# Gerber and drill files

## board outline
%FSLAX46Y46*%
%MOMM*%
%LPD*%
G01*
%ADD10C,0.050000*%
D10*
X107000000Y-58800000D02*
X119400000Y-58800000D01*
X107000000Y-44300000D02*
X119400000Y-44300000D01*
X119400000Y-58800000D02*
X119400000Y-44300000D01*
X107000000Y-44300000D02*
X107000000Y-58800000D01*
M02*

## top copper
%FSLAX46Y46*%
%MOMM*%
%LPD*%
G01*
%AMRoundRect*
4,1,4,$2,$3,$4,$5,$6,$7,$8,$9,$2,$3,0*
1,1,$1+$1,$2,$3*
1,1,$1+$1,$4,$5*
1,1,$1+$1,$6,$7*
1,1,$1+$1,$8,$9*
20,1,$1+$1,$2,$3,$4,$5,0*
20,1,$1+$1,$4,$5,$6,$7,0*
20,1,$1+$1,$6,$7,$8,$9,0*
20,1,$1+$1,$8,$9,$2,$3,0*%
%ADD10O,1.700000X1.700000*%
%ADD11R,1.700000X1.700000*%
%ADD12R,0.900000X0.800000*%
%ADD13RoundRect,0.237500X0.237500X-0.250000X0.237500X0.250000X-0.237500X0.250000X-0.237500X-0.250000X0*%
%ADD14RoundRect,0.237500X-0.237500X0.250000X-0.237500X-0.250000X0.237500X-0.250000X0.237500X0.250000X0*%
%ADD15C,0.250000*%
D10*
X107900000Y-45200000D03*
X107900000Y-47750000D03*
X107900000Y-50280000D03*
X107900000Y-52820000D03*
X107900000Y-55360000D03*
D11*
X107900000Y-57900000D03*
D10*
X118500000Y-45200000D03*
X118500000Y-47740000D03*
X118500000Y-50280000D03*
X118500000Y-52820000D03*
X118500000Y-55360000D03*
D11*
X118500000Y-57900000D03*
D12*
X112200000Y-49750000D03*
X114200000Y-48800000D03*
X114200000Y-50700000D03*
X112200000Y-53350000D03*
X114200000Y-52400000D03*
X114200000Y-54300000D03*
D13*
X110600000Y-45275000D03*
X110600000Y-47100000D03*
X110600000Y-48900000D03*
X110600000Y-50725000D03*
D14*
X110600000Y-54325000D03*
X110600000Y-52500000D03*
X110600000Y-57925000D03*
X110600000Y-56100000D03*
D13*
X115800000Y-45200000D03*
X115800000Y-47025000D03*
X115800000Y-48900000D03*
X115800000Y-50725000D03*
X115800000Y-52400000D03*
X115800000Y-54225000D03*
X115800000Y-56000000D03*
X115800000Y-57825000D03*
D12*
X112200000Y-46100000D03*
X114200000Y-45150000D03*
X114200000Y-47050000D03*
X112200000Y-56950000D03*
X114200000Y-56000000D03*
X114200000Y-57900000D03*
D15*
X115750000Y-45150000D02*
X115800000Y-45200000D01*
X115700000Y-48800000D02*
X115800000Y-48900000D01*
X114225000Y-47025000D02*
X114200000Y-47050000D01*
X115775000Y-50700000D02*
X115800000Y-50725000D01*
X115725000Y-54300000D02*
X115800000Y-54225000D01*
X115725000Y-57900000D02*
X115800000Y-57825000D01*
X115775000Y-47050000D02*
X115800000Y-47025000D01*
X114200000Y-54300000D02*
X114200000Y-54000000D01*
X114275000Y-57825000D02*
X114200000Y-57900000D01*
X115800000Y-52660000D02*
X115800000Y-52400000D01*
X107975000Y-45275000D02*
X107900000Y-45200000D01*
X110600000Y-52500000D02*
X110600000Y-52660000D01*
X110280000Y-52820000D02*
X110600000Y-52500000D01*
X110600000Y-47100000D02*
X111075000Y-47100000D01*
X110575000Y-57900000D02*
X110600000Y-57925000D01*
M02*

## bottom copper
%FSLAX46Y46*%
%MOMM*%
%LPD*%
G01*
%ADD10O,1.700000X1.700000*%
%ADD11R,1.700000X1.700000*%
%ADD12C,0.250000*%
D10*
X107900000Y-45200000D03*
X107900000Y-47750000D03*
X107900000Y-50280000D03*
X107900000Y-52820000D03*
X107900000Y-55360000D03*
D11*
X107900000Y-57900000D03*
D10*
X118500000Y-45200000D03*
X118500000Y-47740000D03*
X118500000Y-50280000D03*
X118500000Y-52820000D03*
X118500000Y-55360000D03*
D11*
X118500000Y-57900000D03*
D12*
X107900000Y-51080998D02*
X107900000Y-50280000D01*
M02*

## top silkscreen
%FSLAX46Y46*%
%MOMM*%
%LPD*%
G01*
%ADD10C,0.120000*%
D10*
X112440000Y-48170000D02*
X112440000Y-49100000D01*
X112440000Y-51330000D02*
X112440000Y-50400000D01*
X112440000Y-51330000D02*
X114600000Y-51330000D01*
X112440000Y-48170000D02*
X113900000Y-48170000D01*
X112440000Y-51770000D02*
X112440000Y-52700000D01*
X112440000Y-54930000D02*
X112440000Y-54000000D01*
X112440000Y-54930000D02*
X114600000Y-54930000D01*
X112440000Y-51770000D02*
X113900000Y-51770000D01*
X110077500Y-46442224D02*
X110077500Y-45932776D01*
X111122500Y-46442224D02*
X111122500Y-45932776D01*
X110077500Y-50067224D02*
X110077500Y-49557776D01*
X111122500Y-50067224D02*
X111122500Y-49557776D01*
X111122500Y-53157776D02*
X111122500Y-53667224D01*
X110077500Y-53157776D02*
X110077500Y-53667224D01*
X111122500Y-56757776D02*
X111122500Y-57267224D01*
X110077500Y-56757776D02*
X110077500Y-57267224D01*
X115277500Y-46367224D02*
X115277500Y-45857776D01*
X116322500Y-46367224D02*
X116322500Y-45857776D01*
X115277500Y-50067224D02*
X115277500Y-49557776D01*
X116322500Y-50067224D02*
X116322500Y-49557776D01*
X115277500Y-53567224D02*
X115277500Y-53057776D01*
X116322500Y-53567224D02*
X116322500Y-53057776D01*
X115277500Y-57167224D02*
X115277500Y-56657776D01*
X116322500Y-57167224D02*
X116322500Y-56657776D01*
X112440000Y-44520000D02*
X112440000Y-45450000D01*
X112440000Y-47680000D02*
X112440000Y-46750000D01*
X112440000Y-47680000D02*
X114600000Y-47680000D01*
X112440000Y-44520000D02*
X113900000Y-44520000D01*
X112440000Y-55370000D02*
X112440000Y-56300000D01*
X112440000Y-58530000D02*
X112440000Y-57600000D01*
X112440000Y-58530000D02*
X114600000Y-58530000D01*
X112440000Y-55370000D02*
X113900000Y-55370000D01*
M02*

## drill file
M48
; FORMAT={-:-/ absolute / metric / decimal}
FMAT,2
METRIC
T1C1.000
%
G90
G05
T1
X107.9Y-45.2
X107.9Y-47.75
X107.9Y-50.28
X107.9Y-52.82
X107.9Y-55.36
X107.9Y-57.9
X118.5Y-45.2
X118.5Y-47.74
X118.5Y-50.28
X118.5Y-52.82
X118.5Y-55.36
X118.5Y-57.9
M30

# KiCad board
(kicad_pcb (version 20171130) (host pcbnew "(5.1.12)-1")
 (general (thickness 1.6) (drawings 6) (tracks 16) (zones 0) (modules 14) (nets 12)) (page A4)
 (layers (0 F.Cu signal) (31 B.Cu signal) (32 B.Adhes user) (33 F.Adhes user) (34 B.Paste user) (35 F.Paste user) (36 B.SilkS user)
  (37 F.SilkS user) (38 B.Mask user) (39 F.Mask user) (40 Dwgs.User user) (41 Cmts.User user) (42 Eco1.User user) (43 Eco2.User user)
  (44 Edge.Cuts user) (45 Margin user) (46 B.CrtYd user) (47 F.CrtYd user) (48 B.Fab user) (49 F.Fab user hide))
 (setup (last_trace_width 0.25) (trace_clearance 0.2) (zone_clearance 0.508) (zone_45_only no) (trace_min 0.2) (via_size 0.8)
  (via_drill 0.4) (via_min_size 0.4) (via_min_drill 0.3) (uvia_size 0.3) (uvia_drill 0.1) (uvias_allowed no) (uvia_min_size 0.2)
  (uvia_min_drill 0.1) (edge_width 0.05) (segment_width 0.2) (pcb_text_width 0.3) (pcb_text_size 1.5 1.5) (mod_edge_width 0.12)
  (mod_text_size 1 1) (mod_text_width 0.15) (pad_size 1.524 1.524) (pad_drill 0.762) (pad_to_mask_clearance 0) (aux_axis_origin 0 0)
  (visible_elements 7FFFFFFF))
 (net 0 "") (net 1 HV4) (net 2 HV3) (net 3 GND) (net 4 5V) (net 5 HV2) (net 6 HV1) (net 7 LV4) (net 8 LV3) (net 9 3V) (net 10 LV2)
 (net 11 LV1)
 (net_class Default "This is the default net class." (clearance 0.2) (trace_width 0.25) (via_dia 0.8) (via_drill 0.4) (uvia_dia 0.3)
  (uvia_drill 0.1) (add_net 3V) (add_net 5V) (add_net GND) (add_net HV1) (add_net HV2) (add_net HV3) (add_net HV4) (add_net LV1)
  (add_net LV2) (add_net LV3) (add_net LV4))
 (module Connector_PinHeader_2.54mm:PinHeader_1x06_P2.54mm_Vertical (layer B.Cu) (at 107.9 57.9)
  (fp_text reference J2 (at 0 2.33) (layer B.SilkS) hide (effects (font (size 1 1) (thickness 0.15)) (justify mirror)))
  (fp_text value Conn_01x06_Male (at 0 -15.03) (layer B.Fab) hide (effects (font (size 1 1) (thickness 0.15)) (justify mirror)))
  (pad 6 thru_hole oval (at 0 -12.7) (size 1.7 1.7) (drill 1) (layers *.Cu *.Mask) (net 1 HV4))
  (pad 5 thru_hole oval (at 0 -10.15) (size 1.7 1.7) (drill 1) (layers *.Cu *.Mask) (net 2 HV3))
  (pad 4 thru_hole oval (at 0 -7.62) (size 1.7 1.7) (drill 1) (layers *.Cu *.Mask) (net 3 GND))
  (pad 3 thru_hole oval (at 0 -5.08) (size 1.7 1.7) (drill 1) (layers *.Cu *.Mask) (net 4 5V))
  (pad 2 thru_hole oval (at 0 -2.54) (size 1.7 1.7) (drill 1) (layers *.Cu *.Mask) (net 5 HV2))
  (pad 1 thru_hole rect (at 0 0) (size 1.7 1.7) (drill 1) (layers *.Cu *.Mask) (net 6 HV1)))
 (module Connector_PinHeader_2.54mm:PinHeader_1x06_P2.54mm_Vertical (layer B.Cu) (at 118.5 57.9)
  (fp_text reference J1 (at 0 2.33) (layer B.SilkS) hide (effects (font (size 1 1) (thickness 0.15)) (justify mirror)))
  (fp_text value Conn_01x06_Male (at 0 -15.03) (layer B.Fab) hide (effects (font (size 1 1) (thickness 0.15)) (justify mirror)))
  (pad 6 thru_hole oval (at 0 -12.7) (size 1.7 1.7) (drill 1) (layers *.Cu *.Mask) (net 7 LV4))
  (pad 5 thru_hole oval (at 0 -10.16) (size 1.7 1.7) (drill 1) (layers *.Cu *.Mask) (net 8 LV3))
  (pad 4 thru_hole oval (at 0 -7.62) (size 1.7 1.7) (drill 1) (layers *.Cu *.Mask) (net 3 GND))
  (pad 3 thru_hole oval (at 0 -5.08) (size 1.7 1.7) (drill 1) (layers *.Cu *.Mask) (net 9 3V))
  (pad 2 thru_hole oval (at 0 -2.54) (size 1.7 1.7) (drill 1) (layers *.Cu *.Mask) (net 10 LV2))
  (pad 1 thru_hole rect (at 0 0) (size 1.7 1.7) (drill 1) (layers *.Cu *.Mask) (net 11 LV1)))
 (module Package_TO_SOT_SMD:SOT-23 (layer F.Cu) (at 113.2 49.75 180)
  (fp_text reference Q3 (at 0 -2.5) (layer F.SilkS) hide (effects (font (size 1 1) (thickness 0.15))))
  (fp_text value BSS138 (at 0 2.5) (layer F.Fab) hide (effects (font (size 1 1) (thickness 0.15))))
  (fp_line (start 0.76 1.58) (end 0.76 0.65) (layer F.SilkS) (width 0.12))
  (fp_line (start 0.76 -1.58) (end 0.76 -0.65) (layer F.SilkS) (width 0.12))
  (fp_line (start 0.76 -1.58) (end -1.4 -1.58) (layer F.SilkS) (width 0.12))
  (fp_line (start 0.76 1.58) (end -0.7 1.58) (layer F.SilkS) (width 0.12))
  (pad 3 smd rect (at 1 0 180) (size 0.9 0.8) (layers F.Cu F.Paste F.Mask) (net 2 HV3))
  (pad 2 smd rect (at -1 0.95 180) (size 0.9 0.8) (layers F.Cu F.Paste F.Mask) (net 8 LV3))
  (pad 1 smd rect (at -1 -0.95 180) (size 0.9 0.8) (layers F.Cu F.Paste F.Mask) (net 9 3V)))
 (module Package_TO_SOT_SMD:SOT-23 (layer F.Cu) (at 113.2 53.35 180)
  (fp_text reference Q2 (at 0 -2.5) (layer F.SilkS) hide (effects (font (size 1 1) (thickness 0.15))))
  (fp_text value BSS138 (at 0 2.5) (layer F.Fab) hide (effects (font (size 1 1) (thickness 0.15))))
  (fp_line (start 0.76 1.58) (end 0.76 0.65) (layer F.SilkS) (width 0.12))
  (fp_line (start 0.76 -1.58) (end 0.76 -0.65) (layer F.SilkS) (width 0.12))
  (fp_line (start 0.76 -1.58) (end -1.4 -1.58) (layer F.SilkS) (width 0.12))
  (fp_line (start 0.76 1.58) (end -0.7 1.58) (layer F.SilkS) (width 0.12))
  (pad 3 smd rect (at 1 0 180) (size 0.9 0.8) (layers F.Cu F.Paste F.Mask) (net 5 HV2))
  (pad 2 smd rect (at -1 0.95 180) (size 0.9 0.8) (layers F.Cu F.Paste F.Mask) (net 10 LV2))
  (pad 1 smd rect (at -1 -0.95 180) (size 0.9 0.8) (layers F.Cu F.Paste F.Mask) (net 9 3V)))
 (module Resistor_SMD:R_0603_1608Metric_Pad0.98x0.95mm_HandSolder (layer F.Cu) (at 110.6 46.1875 90)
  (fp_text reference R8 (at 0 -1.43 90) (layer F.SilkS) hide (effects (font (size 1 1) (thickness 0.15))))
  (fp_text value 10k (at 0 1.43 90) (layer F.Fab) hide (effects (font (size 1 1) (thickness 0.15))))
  (fp_line (start -0.254724 -0.5225) (end 0.254724 -0.5225) (layer F.SilkS) (width 0.12))
  (fp_line (start -0.254724 0.5225) (end 0.254724 0.5225) (layer F.SilkS) (width 0.12))
  (pad 2 smd roundrect (at 0.9125 0 90) (size 0.975 0.95) (layers F.Cu F.Paste F.Mask) (roundrect_rratio 0.25) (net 1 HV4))
  (pad 1 smd roundrect (at -0.9125 0 90) (size 0.975 0.95) (layers F.Cu F.Paste F.Mask) (roundrect_rratio 0.25) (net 4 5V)))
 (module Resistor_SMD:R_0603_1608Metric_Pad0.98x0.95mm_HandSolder (layer F.Cu) (at 110.6 49.8125 90)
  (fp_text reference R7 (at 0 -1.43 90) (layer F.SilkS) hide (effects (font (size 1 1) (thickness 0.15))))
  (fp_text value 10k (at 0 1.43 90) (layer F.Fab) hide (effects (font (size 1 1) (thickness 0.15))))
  (fp_line (start -0.254724 -0.5225) (end 0.254724 -0.5225) (layer F.SilkS) (width 0.12))
  (fp_line (start -0.254724 0.5225) (end 0.254724 0.5225) (layer F.SilkS) (width 0.12))
  (pad 2 smd roundrect (at 0.9125 0 90) (size 0.975 0.95) (layers F.Cu F.Paste F.Mask) (roundrect_rratio 0.25) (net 2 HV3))
  (pad 1 smd roundrect (at -0.9125 0 90) (size 0.975 0.95) (layers F.Cu F.Paste F.Mask) (roundrect_rratio 0.25) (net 4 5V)))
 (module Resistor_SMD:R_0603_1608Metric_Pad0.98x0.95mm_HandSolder (layer F.Cu) (at 110.6 53.4125 270)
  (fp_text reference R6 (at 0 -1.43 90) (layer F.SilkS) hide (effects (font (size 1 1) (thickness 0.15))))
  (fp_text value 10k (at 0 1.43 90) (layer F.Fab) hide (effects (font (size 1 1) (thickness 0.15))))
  (fp_line (start -0.254724 -0.5225) (end 0.254724 -0.5225) (layer F.SilkS) (width 0.12))
  (fp_line (start -0.254724 0.5225) (end 0.254724 0.5225) (layer F.SilkS) (width 0.12))
  (pad 2 smd roundrect (at 0.9125 0 270) (size 0.975 0.95) (layers F.Cu F.Paste F.Mask) (roundrect_rratio 0.25) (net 5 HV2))
  (pad 1 smd roundrect (at -0.9125 0 270) (size 0.975 0.95) (layers F.Cu F.Paste F.Mask) (roundrect_rratio 0.25) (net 4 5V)))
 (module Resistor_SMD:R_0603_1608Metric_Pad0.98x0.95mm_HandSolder (layer F.Cu) (at 110.6 57.0125 270)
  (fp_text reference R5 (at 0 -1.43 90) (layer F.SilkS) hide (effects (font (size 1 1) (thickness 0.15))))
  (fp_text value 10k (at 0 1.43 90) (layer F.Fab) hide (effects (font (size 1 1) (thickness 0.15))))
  (fp_line (start -0.254724 -0.5225) (end 0.254724 -0.5225) (layer F.SilkS) (width 0.12))
  (fp_line (start -0.254724 0.5225) (end 0.254724 0.5225) (layer F.SilkS) (width 0.12))
  (pad 2 smd roundrect (at 0.9125 0 270) (size 0.975 0.95) (layers F.Cu F.Paste F.Mask) (roundrect_rratio 0.25) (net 6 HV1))
  (pad 1 smd roundrect (at -0.9125 0 270) (size 0.975 0.95) (layers F.Cu F.Paste F.Mask) (roundrect_rratio 0.25) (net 4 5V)))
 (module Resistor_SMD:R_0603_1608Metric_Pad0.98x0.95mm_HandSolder (layer F.Cu) (at 115.8 46.1125 90)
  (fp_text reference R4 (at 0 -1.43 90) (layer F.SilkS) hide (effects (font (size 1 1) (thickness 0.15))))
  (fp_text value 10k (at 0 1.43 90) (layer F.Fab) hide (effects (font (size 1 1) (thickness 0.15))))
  (fp_line (start -0.254724 -0.5225) (end 0.254724 -0.5225) (layer F.SilkS) (width 0.12))
  (fp_line (start -0.254724 0.5225) (end 0.254724 0.5225) (layer F.SilkS) (width 0.12))
  (pad 2 smd roundrect (at 0.9125 0 90) (size 0.975 0.95) (layers F.Cu F.Paste F.Mask) (roundrect_rratio 0.25) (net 7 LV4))
  (pad 1 smd roundrect (at -0.9125 0 90) (size 0.975 0.95) (layers F.Cu F.Paste F.Mask) (roundrect_rratio 0.25) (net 9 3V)))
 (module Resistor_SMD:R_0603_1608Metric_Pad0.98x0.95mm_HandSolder (layer F.Cu) (at 115.8 49.8125 90)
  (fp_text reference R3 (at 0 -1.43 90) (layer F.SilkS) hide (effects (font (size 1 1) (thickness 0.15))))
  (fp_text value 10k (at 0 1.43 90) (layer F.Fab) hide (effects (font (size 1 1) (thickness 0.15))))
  (fp_line (start -0.254724 -0.5225) (end 0.254724 -0.5225) (layer F.SilkS) (width 0.12))
  (fp_line (start -0.254724 0.5225) (end 0.254724 0.5225) (layer F.SilkS) (width 0.12))
  (pad 2 smd roundrect (at 0.9125 0 90) (size 0.975 0.95) (layers F.Cu F.Paste F.Mask) (roundrect_rratio 0.25) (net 8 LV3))
  (pad 1 smd roundrect (at -0.9125 0 90) (size 0.975 0.95) (layers F.Cu F.Paste F.Mask) (roundrect_rratio 0.25) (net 9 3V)))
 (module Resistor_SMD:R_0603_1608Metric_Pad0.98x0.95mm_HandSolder (layer F.Cu) (at 115.8 53.3125 90)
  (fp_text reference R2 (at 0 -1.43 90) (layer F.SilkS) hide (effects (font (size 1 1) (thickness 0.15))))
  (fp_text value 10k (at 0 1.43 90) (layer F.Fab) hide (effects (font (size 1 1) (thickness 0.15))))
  (fp_line (start -0.254724 -0.5225) (end 0.254724 -0.5225) (layer F.SilkS) (width 0.12))
  (fp_line (start -0.254724 0.5225) (end 0.254724 0.5225) (layer F.SilkS) (width 0.12))
  (pad 2 smd roundrect (at 0.9125 0 90) (size 0.975 0.95) (layers F.Cu F.Paste F.Mask) (roundrect_rratio 0.25) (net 10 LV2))
  (pad 1 smd roundrect (at -0.9125 0 90) (size 0.975 0.95) (layers F.Cu F.Paste F.Mask) (roundrect_rratio 0.25) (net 9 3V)))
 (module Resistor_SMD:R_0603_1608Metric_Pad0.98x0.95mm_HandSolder (layer F.Cu) (at 115.8 56.9125 90)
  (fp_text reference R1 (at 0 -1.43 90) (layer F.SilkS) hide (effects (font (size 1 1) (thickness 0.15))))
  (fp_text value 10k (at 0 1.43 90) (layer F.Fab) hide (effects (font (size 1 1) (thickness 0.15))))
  (fp_line (start -0.254724 -0.5225) (end 0.254724 -0.5225) (layer F.SilkS) (width 0.12))
  (fp_line (start -0.254724 0.5225) (end 0.254724 0.5225) (layer F.SilkS) (width 0.12))
  (pad 2 smd roundrect (at 0.9125 0 90) (size 0.975 0.95) (layers F.Cu F.Paste F.Mask) (roundrect_rratio 0.25) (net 11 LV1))
  (pad 1 smd roundrect (at -0.9125 0 90) (size 0.975 0.95) (layers F.Cu F.Paste F.Mask) (roundrect_rratio 0.25) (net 9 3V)))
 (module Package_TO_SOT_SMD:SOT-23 (layer F.Cu) (at 113.2 46.1 180)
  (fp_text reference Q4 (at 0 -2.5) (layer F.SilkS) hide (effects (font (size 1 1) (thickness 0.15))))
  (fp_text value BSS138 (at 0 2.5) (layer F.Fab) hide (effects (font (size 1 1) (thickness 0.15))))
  (fp_line (start 0.76 1.58) (end 0.76 0.65) (layer F.SilkS) (width 0.12))
  (fp_line (start 0.76 -1.58) (end 0.76 -0.65) (layer F.SilkS) (width 0.12))
  (fp_line (start 0.76 -1.58) (end -1.4 -1.58) (layer F.SilkS) (width 0.12))
  (fp_line (start 0.76 1.58) (end -0.7 1.58) (layer F.SilkS) (width 0.12))
  (pad 3 smd rect (at 1 0 180) (size 0.9 0.8) (layers F.Cu F.Paste F.Mask) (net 1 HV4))
  (pad 2 smd rect (at -1 0.95 180) (size 0.9 0.8) (layers F.Cu F.Paste F.Mask) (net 7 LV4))
  (pad 1 smd rect (at -1 -0.95 180) (size 0.9 0.8) (layers F.Cu F.Paste F.Mask) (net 9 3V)))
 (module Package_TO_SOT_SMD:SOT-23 (layer F.Cu) (at 113.2 56.95 180)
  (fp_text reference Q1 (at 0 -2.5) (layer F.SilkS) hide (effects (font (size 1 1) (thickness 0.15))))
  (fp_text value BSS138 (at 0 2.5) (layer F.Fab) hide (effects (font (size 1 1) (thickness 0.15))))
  (fp_line (start 0.76 1.58) (end 0.76 0.65) (layer F.SilkS) (width 0.12))
  (fp_line (start 0.76 -1.58) (end 0.76 -0.65) (layer F.SilkS) (width 0.12))
  (fp_line (start 0.76 -1.58) (end -1.4 -1.58) (layer F.SilkS) (width 0.12))
  (fp_line (start 0.76 1.58) (end -0.7 1.58) (layer F.SilkS) (width 0.12))
  (pad 3 smd rect (at 1 0 180) (size 0.9 0.8) (layers F.Cu F.Paste F.Mask) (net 6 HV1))
  (pad 2 smd rect (at -1 0.95 180) (size 0.9 0.8) (layers F.Cu F.Paste F.Mask) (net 11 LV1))
  (pad 1 smd rect (at -1 -0.95 180) (size 0.9 0.8) (layers F.Cu F.Paste F.Mask) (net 9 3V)))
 (gr_line (start 107 58.8) (end 119.4 58.8) (layer Edge.Cuts) (width 0.05))
 (gr_line (start 107 44.3) (end 119.4 44.3) (layer Edge.Cuts) (width 0.05))
 (gr_line (start 119.4 58.8) (end 119.4 44.3) (layer Edge.Cuts) (width 0.05))
 (gr_line (start 107 44.3) (end 107 58.8) (layer Edge.Cuts) (width 0.05))
 (segment (start 115.75 45.15) (end 115.8 45.2) (width 0.25) (layer F.Cu) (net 7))
 (segment (start 115.7 48.8) (end 115.8 48.9) (width 0.25) (layer F.Cu) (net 8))
 (segment (start 107.9 51.080998) (end 107.9 50.28) (width 0.25) (layer B.Cu) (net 3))
 (segment (start 114.225 47.025) (end 114.2 47.05) (width 0.25) (layer F.Cu) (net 9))
 (segment (start 115.775 50.7) (end 115.8 50.725) (width 0.25) (layer F.Cu) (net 9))
 (segment (start 115.725 54.3) (end 115.8 54.225) (width 0.25) (layer F.Cu) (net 9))
 (segment (start 115.725 57.9) (end 115.8 57.825) (width 0.25) (layer F.Cu) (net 9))
 (segment (start 115.775 47.05) (end 115.8 47.025) (width 0.25) (layer F.Cu) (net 9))
 (segment (start 114.2 54.3) (end 114.2 54) (width 0.25) (layer F.Cu) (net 9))
 (segment (start 114.275 57.825) (end 114.2 57.9) (width 0.25) (layer F.Cu) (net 9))
 (segment (start 115.8 52.66) (end 115.8 52.4) (width 0.25) (layer F.Cu) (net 10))
 (segment (start 107.975 45.275) (end 107.9 45.2) (width 0.25) (layer F.Cu) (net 1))
 (segment (start 110.6 52.5) (end 110.6 52.66) (width 0.25) (layer F.Cu) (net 4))
 (segment (start 110.28 52.82) (end 110.6 52.5) (width 0.25) (layer F.Cu) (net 4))
 (segment (start 110.6 47.1) (end 111.075 47.1) (width 0.25) (layer F.Cu) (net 4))
 (segment (start 110.575 57.9) (end 110.6 57.925) (width 0.25) (layer F.Cu) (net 6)))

